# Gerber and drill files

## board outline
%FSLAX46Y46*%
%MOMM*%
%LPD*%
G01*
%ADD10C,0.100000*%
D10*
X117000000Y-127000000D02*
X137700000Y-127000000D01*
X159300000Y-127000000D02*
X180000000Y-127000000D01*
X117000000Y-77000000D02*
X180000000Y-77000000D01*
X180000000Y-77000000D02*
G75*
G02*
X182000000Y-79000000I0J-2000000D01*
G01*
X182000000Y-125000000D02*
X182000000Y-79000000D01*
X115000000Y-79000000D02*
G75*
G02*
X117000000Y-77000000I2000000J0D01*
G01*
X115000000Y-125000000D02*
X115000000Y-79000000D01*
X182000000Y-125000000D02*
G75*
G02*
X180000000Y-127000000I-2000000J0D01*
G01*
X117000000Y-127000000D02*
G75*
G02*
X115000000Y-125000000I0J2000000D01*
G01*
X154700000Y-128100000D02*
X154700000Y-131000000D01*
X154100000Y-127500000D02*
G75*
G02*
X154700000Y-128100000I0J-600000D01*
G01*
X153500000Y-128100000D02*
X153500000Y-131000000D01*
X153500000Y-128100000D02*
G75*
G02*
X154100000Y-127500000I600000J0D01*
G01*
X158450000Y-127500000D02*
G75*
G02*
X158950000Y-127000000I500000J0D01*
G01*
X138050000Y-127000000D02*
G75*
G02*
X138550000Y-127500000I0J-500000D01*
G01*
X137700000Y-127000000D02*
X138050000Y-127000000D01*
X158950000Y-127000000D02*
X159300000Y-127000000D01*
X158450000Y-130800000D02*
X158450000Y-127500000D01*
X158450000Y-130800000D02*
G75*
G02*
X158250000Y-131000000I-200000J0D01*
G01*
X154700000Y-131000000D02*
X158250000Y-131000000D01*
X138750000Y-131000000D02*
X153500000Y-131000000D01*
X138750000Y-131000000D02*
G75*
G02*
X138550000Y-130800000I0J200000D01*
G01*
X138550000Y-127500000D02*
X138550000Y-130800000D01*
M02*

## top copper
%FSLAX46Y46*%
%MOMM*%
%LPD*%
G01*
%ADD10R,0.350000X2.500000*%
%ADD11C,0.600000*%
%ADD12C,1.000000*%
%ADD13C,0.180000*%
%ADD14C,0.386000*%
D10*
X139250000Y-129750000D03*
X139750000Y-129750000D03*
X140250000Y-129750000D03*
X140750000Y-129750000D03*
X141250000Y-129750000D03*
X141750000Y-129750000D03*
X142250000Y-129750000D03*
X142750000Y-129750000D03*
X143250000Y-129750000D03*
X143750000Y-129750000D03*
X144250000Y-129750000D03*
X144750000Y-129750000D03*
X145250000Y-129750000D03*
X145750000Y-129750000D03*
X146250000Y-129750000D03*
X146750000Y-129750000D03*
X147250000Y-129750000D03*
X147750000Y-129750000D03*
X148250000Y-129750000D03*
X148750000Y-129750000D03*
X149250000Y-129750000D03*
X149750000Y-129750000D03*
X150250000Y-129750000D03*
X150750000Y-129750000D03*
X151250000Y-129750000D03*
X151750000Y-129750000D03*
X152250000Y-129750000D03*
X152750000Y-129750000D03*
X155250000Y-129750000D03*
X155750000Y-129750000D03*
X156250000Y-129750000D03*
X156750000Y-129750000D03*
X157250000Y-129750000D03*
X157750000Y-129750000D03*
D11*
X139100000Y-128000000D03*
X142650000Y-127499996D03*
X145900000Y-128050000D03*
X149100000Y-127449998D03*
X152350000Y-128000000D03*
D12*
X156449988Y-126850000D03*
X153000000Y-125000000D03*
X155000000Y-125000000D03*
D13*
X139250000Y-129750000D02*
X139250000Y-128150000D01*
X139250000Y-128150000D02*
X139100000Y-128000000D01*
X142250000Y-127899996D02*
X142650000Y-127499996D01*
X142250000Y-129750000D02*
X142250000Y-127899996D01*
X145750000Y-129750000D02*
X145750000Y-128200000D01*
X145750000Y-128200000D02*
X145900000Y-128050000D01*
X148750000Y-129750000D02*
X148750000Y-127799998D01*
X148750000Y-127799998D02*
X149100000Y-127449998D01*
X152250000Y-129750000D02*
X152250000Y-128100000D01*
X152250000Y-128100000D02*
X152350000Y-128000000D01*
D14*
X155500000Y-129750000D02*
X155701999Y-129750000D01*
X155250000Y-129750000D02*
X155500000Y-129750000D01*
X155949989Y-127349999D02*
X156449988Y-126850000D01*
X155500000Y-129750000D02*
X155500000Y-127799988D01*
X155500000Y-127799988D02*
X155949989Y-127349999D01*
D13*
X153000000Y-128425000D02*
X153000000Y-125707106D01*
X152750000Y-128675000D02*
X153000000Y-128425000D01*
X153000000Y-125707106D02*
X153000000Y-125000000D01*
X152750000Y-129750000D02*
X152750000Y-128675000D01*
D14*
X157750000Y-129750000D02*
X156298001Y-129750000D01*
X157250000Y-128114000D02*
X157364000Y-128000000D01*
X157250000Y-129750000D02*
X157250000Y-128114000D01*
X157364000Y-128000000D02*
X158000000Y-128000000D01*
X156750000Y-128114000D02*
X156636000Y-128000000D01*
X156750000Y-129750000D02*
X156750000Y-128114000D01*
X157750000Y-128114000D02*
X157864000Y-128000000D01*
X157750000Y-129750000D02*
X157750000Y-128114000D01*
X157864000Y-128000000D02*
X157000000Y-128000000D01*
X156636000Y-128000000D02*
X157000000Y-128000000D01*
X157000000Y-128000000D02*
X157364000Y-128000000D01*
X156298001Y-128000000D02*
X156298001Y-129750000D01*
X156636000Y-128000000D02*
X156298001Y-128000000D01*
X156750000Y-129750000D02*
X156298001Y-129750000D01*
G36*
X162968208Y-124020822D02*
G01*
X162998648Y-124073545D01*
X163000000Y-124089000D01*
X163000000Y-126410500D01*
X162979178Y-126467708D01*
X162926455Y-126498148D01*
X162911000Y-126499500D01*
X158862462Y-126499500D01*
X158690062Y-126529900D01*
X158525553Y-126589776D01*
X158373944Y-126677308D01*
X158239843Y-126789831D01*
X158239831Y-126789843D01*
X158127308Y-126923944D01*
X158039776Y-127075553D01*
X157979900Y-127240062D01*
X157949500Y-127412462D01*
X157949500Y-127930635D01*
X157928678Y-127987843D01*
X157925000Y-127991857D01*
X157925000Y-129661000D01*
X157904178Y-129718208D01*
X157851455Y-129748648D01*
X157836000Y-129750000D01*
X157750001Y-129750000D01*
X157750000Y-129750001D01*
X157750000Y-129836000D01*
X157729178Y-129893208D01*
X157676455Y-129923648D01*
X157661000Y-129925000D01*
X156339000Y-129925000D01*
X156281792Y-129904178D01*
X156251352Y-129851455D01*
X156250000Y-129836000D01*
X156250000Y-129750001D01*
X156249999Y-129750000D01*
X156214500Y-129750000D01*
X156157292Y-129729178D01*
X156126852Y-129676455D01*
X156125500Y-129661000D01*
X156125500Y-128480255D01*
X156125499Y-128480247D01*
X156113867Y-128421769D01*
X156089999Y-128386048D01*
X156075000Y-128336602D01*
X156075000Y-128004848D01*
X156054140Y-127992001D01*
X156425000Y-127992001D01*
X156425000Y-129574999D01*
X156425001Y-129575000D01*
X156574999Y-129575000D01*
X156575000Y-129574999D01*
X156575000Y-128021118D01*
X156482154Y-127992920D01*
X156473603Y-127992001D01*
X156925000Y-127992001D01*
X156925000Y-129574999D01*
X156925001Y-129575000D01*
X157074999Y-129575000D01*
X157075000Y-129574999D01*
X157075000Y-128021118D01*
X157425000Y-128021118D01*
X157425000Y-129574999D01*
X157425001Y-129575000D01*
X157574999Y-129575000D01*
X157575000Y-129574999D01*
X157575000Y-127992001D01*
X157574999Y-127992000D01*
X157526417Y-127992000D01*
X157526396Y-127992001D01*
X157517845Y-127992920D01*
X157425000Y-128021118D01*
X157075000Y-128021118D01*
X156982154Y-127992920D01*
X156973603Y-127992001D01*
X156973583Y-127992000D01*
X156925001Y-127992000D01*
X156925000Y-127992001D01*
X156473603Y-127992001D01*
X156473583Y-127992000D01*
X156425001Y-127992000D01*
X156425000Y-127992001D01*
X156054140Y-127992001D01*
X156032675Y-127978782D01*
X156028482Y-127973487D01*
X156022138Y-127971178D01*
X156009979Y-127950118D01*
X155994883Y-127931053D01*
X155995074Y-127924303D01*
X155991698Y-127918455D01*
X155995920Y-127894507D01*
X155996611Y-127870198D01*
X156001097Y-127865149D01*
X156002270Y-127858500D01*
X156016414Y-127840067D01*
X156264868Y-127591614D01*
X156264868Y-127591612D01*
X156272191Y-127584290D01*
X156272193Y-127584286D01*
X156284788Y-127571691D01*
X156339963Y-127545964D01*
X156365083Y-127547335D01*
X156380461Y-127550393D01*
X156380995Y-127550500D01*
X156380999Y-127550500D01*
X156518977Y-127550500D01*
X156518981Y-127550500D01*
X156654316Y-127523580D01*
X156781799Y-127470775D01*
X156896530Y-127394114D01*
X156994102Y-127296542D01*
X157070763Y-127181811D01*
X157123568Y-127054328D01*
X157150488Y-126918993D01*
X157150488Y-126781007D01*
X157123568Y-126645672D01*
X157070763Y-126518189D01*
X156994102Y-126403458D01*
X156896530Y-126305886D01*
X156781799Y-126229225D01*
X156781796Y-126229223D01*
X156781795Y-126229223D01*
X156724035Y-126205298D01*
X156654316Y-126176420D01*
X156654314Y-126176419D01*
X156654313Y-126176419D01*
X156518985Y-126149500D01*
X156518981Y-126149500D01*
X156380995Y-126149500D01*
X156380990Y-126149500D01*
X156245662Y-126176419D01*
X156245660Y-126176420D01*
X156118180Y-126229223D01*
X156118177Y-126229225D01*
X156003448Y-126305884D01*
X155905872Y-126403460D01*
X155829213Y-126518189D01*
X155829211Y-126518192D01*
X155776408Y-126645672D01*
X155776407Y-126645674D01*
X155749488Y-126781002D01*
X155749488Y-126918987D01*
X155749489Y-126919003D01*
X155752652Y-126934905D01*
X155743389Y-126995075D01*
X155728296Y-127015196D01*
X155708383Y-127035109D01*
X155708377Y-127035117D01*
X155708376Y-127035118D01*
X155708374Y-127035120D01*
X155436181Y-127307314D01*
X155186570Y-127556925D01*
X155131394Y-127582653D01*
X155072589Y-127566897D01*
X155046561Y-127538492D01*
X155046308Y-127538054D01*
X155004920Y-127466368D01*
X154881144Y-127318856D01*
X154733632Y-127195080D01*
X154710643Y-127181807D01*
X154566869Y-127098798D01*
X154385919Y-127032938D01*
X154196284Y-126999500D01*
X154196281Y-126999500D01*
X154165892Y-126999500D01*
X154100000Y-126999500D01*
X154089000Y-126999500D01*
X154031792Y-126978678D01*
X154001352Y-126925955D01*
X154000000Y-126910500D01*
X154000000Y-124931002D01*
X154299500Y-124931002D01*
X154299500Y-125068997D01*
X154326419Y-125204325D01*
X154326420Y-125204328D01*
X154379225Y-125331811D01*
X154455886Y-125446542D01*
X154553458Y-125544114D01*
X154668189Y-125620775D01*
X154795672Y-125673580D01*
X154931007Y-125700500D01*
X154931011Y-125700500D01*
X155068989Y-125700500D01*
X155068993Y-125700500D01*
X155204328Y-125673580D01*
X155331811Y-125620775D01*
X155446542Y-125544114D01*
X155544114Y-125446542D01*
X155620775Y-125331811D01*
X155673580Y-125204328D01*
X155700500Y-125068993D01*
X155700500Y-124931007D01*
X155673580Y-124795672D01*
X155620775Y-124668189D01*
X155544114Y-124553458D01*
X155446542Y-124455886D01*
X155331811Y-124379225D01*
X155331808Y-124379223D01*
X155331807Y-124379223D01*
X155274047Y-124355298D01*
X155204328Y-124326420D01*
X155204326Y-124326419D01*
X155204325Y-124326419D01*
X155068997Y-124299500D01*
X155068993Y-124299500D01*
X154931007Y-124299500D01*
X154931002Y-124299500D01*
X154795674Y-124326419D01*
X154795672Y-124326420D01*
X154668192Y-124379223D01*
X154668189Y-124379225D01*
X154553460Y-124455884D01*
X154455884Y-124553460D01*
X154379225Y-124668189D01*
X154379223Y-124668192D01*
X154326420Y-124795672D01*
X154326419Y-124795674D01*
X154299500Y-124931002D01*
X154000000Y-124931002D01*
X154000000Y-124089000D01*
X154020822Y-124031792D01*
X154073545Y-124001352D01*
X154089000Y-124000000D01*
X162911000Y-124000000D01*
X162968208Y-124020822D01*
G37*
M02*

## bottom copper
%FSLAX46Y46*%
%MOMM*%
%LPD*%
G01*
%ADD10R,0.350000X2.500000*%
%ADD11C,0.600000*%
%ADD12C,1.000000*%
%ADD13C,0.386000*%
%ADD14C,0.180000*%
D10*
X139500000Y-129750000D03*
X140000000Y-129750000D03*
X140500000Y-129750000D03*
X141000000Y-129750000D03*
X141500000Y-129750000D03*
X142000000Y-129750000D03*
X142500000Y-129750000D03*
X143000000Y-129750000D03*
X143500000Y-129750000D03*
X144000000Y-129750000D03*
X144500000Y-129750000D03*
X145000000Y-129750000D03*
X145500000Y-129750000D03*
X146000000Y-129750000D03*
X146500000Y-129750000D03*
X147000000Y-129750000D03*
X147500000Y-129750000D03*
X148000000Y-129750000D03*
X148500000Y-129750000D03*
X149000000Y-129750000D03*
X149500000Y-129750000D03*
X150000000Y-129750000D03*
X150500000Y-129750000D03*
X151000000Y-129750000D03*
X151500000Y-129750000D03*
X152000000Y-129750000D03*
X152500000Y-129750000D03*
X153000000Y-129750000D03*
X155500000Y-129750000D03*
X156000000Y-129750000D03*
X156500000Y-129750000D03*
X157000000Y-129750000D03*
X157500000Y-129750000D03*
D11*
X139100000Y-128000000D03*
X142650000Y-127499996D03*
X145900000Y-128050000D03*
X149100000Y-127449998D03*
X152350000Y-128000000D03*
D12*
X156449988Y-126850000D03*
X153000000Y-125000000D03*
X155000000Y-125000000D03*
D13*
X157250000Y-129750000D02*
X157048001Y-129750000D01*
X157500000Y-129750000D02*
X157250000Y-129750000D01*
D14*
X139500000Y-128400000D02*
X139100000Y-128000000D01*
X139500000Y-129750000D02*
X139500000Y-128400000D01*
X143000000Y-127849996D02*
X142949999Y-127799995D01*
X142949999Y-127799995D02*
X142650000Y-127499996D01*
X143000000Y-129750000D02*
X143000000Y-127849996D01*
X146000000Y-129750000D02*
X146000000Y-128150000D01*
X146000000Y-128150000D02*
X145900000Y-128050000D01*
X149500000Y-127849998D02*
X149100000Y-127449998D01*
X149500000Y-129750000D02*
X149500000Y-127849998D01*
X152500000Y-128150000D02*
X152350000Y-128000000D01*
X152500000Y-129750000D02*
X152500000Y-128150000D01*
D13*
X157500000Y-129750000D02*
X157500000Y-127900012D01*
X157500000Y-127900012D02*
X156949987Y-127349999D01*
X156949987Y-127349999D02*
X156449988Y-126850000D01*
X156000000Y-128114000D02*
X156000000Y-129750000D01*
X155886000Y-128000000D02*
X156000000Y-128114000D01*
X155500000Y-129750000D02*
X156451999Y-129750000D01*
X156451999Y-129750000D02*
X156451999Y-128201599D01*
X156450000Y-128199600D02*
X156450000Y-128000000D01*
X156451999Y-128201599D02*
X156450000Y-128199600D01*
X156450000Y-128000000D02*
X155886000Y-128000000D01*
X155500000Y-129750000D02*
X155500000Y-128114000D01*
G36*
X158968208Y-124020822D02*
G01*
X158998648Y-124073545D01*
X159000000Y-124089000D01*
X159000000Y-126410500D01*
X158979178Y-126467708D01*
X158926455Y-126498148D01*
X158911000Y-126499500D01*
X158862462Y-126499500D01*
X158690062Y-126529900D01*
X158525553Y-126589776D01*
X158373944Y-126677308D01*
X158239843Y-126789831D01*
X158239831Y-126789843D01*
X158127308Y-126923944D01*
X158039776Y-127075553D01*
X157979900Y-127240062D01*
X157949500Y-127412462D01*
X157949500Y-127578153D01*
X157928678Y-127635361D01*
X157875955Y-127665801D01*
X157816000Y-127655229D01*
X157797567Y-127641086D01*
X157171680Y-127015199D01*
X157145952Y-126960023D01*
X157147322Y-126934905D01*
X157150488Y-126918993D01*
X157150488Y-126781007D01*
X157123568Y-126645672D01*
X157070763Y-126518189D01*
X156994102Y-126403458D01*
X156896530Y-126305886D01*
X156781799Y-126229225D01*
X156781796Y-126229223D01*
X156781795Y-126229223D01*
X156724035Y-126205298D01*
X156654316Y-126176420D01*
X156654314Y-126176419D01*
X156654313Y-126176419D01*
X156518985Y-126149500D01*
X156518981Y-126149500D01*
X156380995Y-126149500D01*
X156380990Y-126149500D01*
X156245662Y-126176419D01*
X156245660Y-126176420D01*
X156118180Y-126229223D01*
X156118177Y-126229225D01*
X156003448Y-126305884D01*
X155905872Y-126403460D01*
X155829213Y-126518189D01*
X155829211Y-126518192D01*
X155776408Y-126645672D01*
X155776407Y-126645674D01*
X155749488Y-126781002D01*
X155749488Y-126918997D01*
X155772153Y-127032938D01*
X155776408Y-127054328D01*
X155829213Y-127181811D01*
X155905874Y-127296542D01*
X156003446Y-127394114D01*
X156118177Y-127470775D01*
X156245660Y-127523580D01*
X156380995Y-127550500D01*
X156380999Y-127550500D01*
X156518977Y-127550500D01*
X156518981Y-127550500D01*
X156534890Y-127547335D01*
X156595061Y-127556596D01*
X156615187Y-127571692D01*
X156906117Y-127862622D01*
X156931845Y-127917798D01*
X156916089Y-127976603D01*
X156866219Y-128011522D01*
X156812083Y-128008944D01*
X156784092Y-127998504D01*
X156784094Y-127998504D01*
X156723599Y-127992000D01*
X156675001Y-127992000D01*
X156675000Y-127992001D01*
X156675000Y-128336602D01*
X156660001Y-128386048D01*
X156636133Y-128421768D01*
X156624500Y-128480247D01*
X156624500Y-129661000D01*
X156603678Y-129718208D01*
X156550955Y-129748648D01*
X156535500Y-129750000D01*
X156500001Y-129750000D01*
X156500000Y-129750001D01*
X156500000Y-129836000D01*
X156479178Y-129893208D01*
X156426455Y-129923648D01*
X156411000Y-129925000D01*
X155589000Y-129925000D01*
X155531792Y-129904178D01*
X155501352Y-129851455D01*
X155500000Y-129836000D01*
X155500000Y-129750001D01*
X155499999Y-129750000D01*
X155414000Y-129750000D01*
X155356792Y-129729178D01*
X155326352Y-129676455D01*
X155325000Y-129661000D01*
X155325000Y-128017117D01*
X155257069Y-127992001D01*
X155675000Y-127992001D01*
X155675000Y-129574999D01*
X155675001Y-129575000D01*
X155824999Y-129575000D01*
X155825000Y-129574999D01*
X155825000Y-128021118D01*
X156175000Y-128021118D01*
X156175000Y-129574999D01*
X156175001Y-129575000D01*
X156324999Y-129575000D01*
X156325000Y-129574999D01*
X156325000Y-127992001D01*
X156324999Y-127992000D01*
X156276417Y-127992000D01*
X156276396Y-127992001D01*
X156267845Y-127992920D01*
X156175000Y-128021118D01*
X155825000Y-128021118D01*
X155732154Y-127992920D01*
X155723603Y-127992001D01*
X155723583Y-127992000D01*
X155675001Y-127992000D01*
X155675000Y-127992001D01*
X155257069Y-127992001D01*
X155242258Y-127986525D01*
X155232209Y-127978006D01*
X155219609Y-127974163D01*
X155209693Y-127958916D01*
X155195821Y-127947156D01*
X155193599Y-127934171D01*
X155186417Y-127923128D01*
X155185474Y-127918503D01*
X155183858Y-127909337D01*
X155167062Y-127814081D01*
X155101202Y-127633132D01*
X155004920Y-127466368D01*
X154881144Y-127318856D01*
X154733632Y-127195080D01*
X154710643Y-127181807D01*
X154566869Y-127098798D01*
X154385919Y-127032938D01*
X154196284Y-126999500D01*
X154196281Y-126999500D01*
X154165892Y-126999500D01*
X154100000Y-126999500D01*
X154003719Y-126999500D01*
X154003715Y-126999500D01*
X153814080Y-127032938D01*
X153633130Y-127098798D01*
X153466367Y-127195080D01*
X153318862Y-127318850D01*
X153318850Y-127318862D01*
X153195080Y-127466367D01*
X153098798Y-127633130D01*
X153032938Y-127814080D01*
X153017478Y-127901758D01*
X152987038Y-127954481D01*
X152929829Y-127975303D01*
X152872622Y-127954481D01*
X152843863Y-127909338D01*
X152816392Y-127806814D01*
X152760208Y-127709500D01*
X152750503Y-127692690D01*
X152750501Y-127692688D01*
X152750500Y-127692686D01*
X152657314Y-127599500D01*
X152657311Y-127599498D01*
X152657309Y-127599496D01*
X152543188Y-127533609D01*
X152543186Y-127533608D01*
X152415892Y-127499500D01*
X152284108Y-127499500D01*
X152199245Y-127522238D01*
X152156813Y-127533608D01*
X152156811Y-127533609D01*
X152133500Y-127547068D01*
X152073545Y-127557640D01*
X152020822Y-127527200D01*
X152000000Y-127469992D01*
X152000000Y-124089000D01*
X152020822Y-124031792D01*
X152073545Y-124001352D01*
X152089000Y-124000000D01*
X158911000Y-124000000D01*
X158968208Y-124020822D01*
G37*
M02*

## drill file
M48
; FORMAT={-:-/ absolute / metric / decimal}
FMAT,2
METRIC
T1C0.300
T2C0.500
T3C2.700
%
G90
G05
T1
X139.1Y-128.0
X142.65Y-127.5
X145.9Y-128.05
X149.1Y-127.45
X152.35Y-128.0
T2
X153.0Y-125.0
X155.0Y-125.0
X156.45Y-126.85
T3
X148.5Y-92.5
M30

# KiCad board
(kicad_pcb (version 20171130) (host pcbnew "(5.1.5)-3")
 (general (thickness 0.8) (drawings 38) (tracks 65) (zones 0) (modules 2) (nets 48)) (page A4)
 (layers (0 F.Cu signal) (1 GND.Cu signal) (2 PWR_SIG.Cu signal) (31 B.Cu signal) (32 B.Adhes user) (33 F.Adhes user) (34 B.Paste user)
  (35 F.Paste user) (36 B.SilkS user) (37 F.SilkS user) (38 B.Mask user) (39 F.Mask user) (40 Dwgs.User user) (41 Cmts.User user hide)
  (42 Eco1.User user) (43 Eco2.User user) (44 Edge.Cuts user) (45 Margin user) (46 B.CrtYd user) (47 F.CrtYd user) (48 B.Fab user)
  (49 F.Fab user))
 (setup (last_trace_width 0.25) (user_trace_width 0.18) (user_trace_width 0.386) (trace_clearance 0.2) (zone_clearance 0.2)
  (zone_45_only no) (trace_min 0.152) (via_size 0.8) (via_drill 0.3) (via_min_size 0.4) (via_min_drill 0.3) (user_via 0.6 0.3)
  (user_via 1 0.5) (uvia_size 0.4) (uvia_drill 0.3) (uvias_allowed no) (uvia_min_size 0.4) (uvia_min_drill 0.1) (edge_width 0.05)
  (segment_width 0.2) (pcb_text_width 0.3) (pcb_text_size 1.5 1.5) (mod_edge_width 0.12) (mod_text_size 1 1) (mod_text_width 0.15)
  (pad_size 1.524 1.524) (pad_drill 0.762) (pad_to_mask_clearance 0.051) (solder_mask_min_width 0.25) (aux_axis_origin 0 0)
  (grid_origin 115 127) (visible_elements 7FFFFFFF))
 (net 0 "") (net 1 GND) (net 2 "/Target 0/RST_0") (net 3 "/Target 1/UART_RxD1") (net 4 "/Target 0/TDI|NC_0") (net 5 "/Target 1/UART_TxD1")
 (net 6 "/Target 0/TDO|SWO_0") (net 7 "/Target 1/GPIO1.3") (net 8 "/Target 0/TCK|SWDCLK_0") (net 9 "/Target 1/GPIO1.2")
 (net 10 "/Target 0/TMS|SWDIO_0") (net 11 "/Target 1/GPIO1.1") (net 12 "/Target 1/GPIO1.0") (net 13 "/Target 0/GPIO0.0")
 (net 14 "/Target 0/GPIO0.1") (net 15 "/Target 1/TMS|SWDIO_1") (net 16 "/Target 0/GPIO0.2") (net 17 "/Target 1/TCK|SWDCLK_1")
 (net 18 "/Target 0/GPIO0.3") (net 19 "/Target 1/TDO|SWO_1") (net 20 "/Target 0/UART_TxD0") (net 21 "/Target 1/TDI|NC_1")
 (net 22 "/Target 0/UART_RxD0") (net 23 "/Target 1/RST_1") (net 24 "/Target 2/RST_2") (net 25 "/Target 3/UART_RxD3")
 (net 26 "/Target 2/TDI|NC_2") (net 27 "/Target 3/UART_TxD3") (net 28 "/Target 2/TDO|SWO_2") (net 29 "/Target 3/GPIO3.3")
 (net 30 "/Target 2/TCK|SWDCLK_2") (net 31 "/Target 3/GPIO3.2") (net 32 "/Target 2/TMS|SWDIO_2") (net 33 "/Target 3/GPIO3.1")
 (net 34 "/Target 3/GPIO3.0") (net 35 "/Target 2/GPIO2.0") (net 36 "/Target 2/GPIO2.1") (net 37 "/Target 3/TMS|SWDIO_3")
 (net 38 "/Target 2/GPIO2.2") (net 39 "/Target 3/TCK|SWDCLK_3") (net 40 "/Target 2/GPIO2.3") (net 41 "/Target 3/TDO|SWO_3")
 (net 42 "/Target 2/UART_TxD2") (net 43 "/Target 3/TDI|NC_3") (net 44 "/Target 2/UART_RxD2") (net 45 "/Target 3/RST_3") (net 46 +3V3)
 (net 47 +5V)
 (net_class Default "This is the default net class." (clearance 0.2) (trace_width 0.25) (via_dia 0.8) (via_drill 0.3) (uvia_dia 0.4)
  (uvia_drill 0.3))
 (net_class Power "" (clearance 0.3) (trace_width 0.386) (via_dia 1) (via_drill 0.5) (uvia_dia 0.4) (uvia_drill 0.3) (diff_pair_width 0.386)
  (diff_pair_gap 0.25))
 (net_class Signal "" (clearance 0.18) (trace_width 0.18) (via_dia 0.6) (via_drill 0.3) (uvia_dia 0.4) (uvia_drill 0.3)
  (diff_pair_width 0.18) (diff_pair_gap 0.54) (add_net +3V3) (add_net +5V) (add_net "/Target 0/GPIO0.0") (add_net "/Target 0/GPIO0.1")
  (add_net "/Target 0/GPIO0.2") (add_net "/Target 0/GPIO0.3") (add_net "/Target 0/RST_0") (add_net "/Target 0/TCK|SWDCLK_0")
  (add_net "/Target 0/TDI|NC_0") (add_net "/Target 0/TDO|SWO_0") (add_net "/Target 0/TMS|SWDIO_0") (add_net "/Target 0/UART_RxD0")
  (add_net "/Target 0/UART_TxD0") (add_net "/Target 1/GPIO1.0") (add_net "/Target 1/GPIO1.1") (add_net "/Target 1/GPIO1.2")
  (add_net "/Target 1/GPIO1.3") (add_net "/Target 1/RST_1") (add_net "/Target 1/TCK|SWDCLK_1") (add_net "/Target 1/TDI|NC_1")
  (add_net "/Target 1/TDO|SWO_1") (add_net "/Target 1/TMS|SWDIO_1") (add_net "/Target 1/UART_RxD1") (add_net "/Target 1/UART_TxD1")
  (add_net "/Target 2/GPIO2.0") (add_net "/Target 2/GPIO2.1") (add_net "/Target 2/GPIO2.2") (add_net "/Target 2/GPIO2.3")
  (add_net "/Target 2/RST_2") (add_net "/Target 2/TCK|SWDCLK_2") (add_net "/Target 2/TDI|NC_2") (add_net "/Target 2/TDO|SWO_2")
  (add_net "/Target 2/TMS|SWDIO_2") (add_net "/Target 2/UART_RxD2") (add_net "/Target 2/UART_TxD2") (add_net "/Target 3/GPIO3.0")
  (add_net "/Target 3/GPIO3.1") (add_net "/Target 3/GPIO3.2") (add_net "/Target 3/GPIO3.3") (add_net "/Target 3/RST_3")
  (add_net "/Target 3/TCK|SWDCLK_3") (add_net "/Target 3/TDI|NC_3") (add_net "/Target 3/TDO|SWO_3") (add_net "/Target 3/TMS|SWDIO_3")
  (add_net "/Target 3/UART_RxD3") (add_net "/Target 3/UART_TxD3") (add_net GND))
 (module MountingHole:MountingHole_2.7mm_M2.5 (layer F.Cu) (at 148.5 92.5)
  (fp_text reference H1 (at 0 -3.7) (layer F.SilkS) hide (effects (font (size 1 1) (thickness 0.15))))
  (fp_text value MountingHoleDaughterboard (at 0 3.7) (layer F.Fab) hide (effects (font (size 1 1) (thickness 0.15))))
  (pad 1 np_thru_hole circle (at 0 0) (size 2.7 2.7) (drill 2.7) (layers *.Cu *.Mask)))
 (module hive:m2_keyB (layer F.Cu) (at 148.5 131)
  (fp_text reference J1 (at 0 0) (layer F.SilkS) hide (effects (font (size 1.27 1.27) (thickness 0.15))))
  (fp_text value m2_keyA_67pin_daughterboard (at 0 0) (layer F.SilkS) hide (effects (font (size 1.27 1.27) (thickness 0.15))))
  (fp_line (start 6.2 -2.9) (end 6.2 0) (layer Edge.Cuts) (width 0.1))
  (fp_arc (start 5.6 -2.9) (end 5.6 -3.5) (angle 90) (layer Edge.Cuts) (width 0.1))
  (fp_line (start 5 -2.9) (end 5 0) (layer Edge.Cuts) (width 0.1))
  (fp_arc (start 5.6 -2.9) (end 5.6 -3.5) (angle -90) (layer Edge.Cuts) (width 0.1))
  (fp_arc (start 10.45 -3.5) (end 9.95 -3.5) (angle 90) (layer Edge.Cuts) (width 0.1))
  (fp_arc (start -10.45 -3.5) (end -10.45 -4) (angle 90) (layer Edge.Cuts) (width 0.1))
  (fp_line (start -10.8 -4) (end -10.45 -4) (layer Edge.Cuts) (width 0.1))
  (fp_line (start 10.45 -4) (end 10.8 -4) (layer Edge.Cuts) (width 0.1))
  (fp_line (start 9.95 -0.2) (end 9.95 -3.5) (layer Edge.Cuts) (width 0.1))
  (fp_arc (start 9.75 -0.2) (end 9.75 0) (angle -90) (layer Edge.Cuts) (width 0.1))
  (fp_line (start 6.2 0) (end 9.75 0) (layer Edge.Cuts) (width 0.1))
  (fp_line (start -9.75 0) (end 5 0) (layer Edge.Cuts) (width 0.1))
  (fp_arc (start -9.75 -0.2) (end -9.95 -0.2) (angle -90) (layer Edge.Cuts) (width 0.1))
  (fp_line (start -9.95 -3.5) (end -9.95 -0.2) (layer Edge.Cuts) (width 0.1))
  (pad 75 smd rect (at -9.25 -1.25) (size 0.35 2.5) (layers F.Cu F.Paste F.Mask) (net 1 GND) (solder_mask_margin 0.1016))
  (pad 74 smd rect (at -9 -1.25) (size 0.35 2.5) (layers B.Cu B.Paste B.Mask) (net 1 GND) (solder_mask_margin 0.1016))
  (pad 73 smd rect (at -8.75 -1.25) (size 0.35 2.5) (layers F.Cu F.Paste F.Mask) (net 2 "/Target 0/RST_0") (solder_mask_margin 0.1016))
  (pad 72 smd rect (at -8.5 -1.25) (size 0.35 2.5) (layers B.Cu B.Paste B.Mask) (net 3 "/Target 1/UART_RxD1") (solder_mask_margin 0.1016))
  (pad 71 smd rect (at -8.25 -1.25) (size 0.35 2.5) (layers F.Cu F.Paste F.Mask) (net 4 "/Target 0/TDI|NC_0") (solder_mask_margin 0.1016))
  (pad 70 smd rect (at -8 -1.25) (size 0.35 2.5) (layers B.Cu B.Paste B.Mask) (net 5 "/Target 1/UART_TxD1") (solder_mask_margin 0.1016))
  (pad 69 smd rect (at -7.75 -1.25) (size 0.35 2.5) (layers F.Cu F.Paste F.Mask) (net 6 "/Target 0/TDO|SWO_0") (solder_mask_margin 0.1016))
  (pad 68 smd rect (at -7.5 -1.25) (size 0.35 2.5) (layers B.Cu B.Paste B.Mask) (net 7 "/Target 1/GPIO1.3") (solder_mask_margin 0.1016))
  (pad 67 smd rect (at -7.25 -1.25) (size 0.35 2.5) (layers F.Cu F.Paste F.Mask) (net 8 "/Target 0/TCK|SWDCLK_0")
   (solder_mask_margin 0.1016))
  (pad 66 smd rect (at -7 -1.25) (size 0.35 2.5) (layers B.Cu B.Paste B.Mask) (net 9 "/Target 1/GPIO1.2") (solder_mask_margin 0.1016))
  (pad 65 smd rect (at -6.75 -1.25) (size 0.35 2.5) (layers F.Cu F.Paste F.Mask) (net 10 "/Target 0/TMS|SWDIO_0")
   (solder_mask_margin 0.1016))
  (pad 64 smd rect (at -6.5 -1.25) (size 0.35 2.5) (layers B.Cu B.Paste B.Mask) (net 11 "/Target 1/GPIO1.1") (solder_mask_margin 0.1016))
  (pad 63 smd rect (at -6.25 -1.25) (size 0.35 2.5) (layers F.Cu F.Paste F.Mask) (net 1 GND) (solder_mask_margin 0.1016))
  (pad 62 smd rect (at -6 -1.25) (size 0.35 2.5) (layers B.Cu B.Paste B.Mask) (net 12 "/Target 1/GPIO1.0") (solder_mask_margin 0.1016))
  (pad 61 smd rect (at -5.75 -1.25) (size 0.35 2.5) (layers F.Cu F.Paste F.Mask) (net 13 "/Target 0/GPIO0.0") (solder_mask_margin 0.1016))
  (pad 60 smd rect (at -5.5 -1.25) (size 0.35 2.5) (layers B.Cu B.Paste B.Mask) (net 1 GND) (solder_mask_margin 0.1016))
  (pad 59 smd rect (at -5.25 -1.25) (size 0.35 2.5) (layers F.Cu F.Paste F.Mask) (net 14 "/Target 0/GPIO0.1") (solder_mask_margin 0.1016))
  (pad 58 smd rect (at -5 -1.25) (size 0.35 2.5) (layers B.Cu B.Paste B.Mask) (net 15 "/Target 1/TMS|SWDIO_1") (solder_mask_margin 0.1016))
  (pad 57 smd rect (at -4.75 -1.25) (size 0.35 2.5) (layers F.Cu F.Paste F.Mask) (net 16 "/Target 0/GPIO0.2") (solder_mask_margin 0.1016))
  (pad 56 smd rect (at -4.5 -1.25) (size 0.35 2.5) (layers B.Cu B.Paste B.Mask) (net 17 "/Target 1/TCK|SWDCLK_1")
   (solder_mask_margin 0.1016))
  (pad 55 smd rect (at -4.25 -1.25) (size 0.35 2.5) (layers F.Cu F.Paste F.Mask) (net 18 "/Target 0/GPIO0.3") (solder_mask_margin 0.1016))
  (pad 54 smd rect (at -4 -1.25) (size 0.35 2.5) (layers B.Cu B.Paste B.Mask) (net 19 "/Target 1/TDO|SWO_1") (solder_mask_margin 0.1016))
  (pad 53 smd rect (at -3.75 -1.25) (size 0.35 2.5) (layers F.Cu F.Paste F.Mask) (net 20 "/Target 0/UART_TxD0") (solder_mask_margin 0.1016))
  (pad 52 smd rect (at -3.5 -1.25) (size 0.35 2.5) (layers B.Cu B.Paste B.Mask) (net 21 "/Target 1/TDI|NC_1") (solder_mask_margin 0.1016))
  (pad 51 smd rect (at -3.25 -1.25) (size 0.35 2.5) (layers F.Cu F.Paste F.Mask) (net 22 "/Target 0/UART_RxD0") (solder_mask_margin 0.1016))
  (pad 50 smd rect (at -3 -1.25) (size 0.35 2.5) (layers B.Cu B.Paste B.Mask) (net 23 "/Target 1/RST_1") (solder_mask_margin 0.1016))
  (pad 49 smd rect (at -2.75 -1.25) (size 0.35 2.5) (layers F.Cu F.Paste F.Mask) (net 1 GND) (solder_mask_margin 0.1016))
  (pad 48 smd rect (at -2.5 -1.25) (size 0.35 2.5) (layers B.Cu B.Paste B.Mask) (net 1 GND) (solder_mask_margin 0.1016))
  (pad 47 smd rect (at -2.25 -1.25) (size 0.35 2.5) (layers F.Cu F.Paste F.Mask) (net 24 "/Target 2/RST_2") (solder_mask_margin 0.1016))
  (pad 46 smd rect (at -2 -1.25) (size 0.35 2.5) (layers B.Cu B.Paste B.Mask) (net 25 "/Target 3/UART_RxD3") (solder_mask_margin 0.1016))
  (pad 45 smd rect (at -1.75 -1.25) (size 0.35 2.5) (layers F.Cu F.Paste F.Mask) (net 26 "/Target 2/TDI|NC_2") (solder_mask_margin 0.1016))
  (pad 44 smd rect (at -1.5 -1.25) (size 0.35 2.5) (layers B.Cu B.Paste B.Mask) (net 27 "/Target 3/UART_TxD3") (solder_mask_margin 0.1016))
  (pad 43 smd rect (at -1.25 -1.25) (size 0.35 2.5) (layers F.Cu F.Paste F.Mask) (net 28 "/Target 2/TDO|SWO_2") (solder_mask_margin 0.1016))
  (pad 42 smd rect (at -1 -1.25) (size 0.35 2.5) (layers B.Cu B.Paste B.Mask) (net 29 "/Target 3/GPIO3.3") (solder_mask_margin 0.1016))
  (pad 41 smd rect (at -0.75 -1.25) (size 0.35 2.5) (layers F.Cu F.Paste F.Mask) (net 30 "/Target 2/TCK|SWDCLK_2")
   (solder_mask_margin 0.1016))
  (pad 40 smd rect (at -0.5 -1.25) (size 0.35 2.5) (layers B.Cu B.Paste B.Mask) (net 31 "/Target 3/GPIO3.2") (solder_mask_margin 0.1016))
  (pad 39 smd rect (at -0.25 -1.25) (size 0.35 2.5) (layers F.Cu F.Paste F.Mask) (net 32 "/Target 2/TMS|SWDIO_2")
   (solder_mask_margin 0.1016))
  (pad 38 smd rect (at 0 -1.25) (size 0.35 2.5) (layers B.Cu B.Paste B.Mask) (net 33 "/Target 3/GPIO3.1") (solder_mask_margin 0.1016))
  (pad 37 smd rect (at 0.25 -1.25) (size 0.35 2.5) (layers F.Cu F.Paste F.Mask) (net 1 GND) (solder_mask_margin 0.1016))
  (pad 36 smd rect (at 0.5 -1.25) (size 0.35 2.5) (layers B.Cu B.Paste B.Mask) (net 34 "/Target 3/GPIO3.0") (solder_mask_margin 0.1016))
  (pad 35 smd rect (at 0.75 -1.25) (size 0.35 2.5) (layers F.Cu F.Paste F.Mask) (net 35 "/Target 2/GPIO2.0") (solder_mask_margin 0.1016))
  (pad 34 smd rect (at 1 -1.25) (size 0.35 2.5) (layers B.Cu B.Paste B.Mask) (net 1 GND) (solder_mask_margin 0.1016))
  (pad 33 smd rect (at 1.25 -1.25) (size 0.35 2.5) (layers F.Cu F.Paste F.Mask) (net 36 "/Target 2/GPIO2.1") (solder_mask_margin 0.1016))
  (pad 32 smd rect (at 1.5 -1.25) (size 0.35 2.5) (layers B.Cu B.Paste B.Mask) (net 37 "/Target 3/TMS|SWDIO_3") (solder_mask_margin 0.1016))
  (pad 31 smd rect (at 1.75 -1.25) (size 0.35 2.5) (layers F.Cu F.Paste F.Mask) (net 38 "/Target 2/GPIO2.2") (solder_mask_margin 0.1016))
  (pad 30 smd rect (at 2 -1.25) (size 0.35 2.5) (layers B.Cu B.Paste B.Mask) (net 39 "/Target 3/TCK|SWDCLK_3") (solder_mask_margin 0.1016))
  (pad 29 smd rect (at 2.25 -1.25) (size 0.35 2.5) (layers F.Cu F.Paste F.Mask) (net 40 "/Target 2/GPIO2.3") (solder_mask_margin 0.1016))
  (pad 28 smd rect (at 2.5 -1.25) (size 0.35 2.5) (layers B.Cu B.Paste B.Mask) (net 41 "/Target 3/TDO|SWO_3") (solder_mask_margin 0.1016))
  (pad 27 smd rect (at 2.75 -1.25) (size 0.35 2.5) (layers F.Cu F.Paste F.Mask) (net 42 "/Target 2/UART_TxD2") (solder_mask_margin 0.1016))
  (pad 26 smd rect (at 3 -1.25) (size 0.35 2.5) (layers B.Cu B.Paste B.Mask) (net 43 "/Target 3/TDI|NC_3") (solder_mask_margin 0.1016))
  (pad 25 smd rect (at 3.25 -1.25) (size 0.35 2.5) (layers F.Cu F.Paste F.Mask) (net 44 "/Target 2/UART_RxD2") (solder_mask_margin 0.1016))
  (pad 24 smd rect (at 3.5 -1.25) (size 0.35 2.5) (layers B.Cu B.Paste B.Mask) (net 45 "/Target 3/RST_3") (solder_mask_margin 0.1016))
  (pad 23 smd rect (at 3.75 -1.25) (size 0.35 2.5) (layers F.Cu F.Paste F.Mask) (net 1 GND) (solder_mask_margin 0.1016))
  (pad 22 smd rect (at 4 -1.25) (size 0.35 2.5) (layers B.Cu B.Paste B.Mask) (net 1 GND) (solder_mask_margin 0.1016))
  (pad 21 smd rect (at 4.25 -1.25) (size 0.35 2.5) (layers F.Cu F.Paste F.Mask) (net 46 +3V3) (solder_mask_margin 0.1016))
  (pad 20 smd rect (at 4.5 -1.25) (size 0.35 2.5) (layers B.Cu B.Paste B.Mask) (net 46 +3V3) (solder_mask_margin 0.1016))
  (pad 11 smd rect (at 6.75 -1.25) (size 0.35 2.5) (layers F.Cu F.Paste F.Mask) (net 1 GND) (solder_mask_margin 0.1016))
  (pad 10 smd rect (at 7 -1.25) (size 0.35 2.5) (layers B.Cu B.Paste B.Mask) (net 46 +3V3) (solder_mask_margin 0.1016))
  (pad 9 smd rect (at 7.25 -1.25) (size 0.35 2.5) (layers F.Cu F.Paste F.Mask) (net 1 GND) (solder_mask_margin 0.1016))
  (pad 8 smd rect (at 7.5 -1.25) (size 0.35 2.5) (layers B.Cu B.Paste B.Mask) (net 46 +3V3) (solder_mask_margin 0.1016))
  (pad 7 smd rect (at 7.75 -1.25) (size 0.35 2.5) (layers F.Cu F.Paste F.Mask) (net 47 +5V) (solder_mask_margin 0.1016))
  (pad 6 smd rect (at 8 -1.25) (size 0.35 2.5) (layers B.Cu B.Paste B.Mask) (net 46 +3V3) (solder_mask_margin 0.1016))
  (pad 5 smd rect (at 8.25 -1.25) (size 0.35 2.5) (layers F.Cu F.Paste F.Mask) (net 47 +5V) (solder_mask_margin 0.1016))
  (pad 4 smd rect (at 8.5 -1.25) (size 0.35 2.5) (layers B.Cu B.Paste B.Mask) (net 1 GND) (solder_mask_margin 0.1016))
  (pad 3 smd rect (at 8.75 -1.25) (size 0.35 2.5) (layers F.Cu F.Paste F.Mask) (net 47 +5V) (solder_mask_margin 0.1016))
  (pad 2 smd rect (at 9 -1.25) (size 0.35 2.5) (layers B.Cu B.Paste B.Mask) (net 1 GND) (solder_mask_margin 0.1016))
  (pad 1 smd rect (at 9.25 -1.25) (size 0.35 2.5) (layers F.Cu F.Paste F.Mask) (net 47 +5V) (solder_mask_margin 0.1016)))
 (gr_line (start 117 127) (end 137.7 127) (layer Edge.Cuts) (width 0.1))
 (gr_line (start 159.3 127) (end 180 127) (layer Edge.Cuts) (width 0.1))
 (gr_line (start 117 77) (end 180 77) (layer Edge.Cuts) (width 0.1))
 (gr_arc (start 180 79) (end 182 79) (angle -90) (layer Edge.Cuts) (width 0.1))
 (gr_line (start 182 125) (end 182 79) (layer Edge.Cuts) (width 0.1))
 (gr_arc (start 117 79) (end 117 77) (angle -90) (layer Edge.Cuts) (width 0.1))
 (gr_line (start 115 125) (end 115 79) (layer Edge.Cuts) (width 0.1))
 (gr_arc (start 180 125) (end 180 127) (angle -90) (layer Edge.Cuts) (width 0.1))
 (gr_arc (start 117 125) (end 115 125) (angle -90) (layer Edge.Cuts) (width 0.1))
 (segment (start 157.25 129.75) (end 157.048001 129.75) (width 0.386) (layer B.Cu) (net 1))
 (segment (start 157.5 129.75) (end 157.25 129.75) (width 0.386) (layer B.Cu) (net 1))
 (via (at 139.1 128) (size 0.6) (drill 0.3) (layers F.Cu B.Cu) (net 1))
 (segment (start 139.25 129.75) (end 139.25 128.15) (width 0.18) (layer F.Cu) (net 1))
 (segment (start 139.25 128.15) (end 139.1 128) (width 0.18) (layer F.Cu) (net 1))
 (segment (start 139.5 128.4) (end 139.1 128) (width 0.18) (layer B.Cu) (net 1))
 (segment (start 139.5 129.75) (end 139.5 128.4) (width 0.18) (layer B.Cu) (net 1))
 (segment (start 143 127.849996) (end 142.949999 127.799995) (width 0.18) (layer B.Cu) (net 1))
 (segment (start 142.949999 127.799995) (end 142.65 127.499996) (width 0.18) (layer B.Cu) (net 1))
 (via (at 142.65 127.499996) (size 0.6) (drill 0.3) (layers F.Cu B.Cu) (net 1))
 (segment (start 143 129.75) (end 143 127.849996) (width 0.18) (layer B.Cu) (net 1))
 (segment (start 142.25 127.899996) (end 142.65 127.499996) (width 0.18) (layer F.Cu) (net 1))
 (segment (start 142.25 129.75) (end 142.25 127.899996) (width 0.18) (layer F.Cu) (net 1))
 (via (at 145.9 128.05) (size 0.6) (drill 0.3) (layers F.Cu B.Cu) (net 1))
 (segment (start 146 129.75) (end 146 128.15) (width 0.18) (layer B.Cu) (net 1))
 (segment (start 145.75 129.75) (end 145.75 128.2) (width 0.18) (layer F.Cu) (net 1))
 (segment (start 146 128.15) (end 145.9 128.05) (width 0.18) (layer B.Cu) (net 1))
 (segment (start 145.75 128.2) (end 145.9 128.05) (width 0.18) (layer F.Cu) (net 1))
 (via (at 149.1 127.449998) (size 0.6) (drill 0.3) (layers F.Cu B.Cu) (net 1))
 (segment (start 149.5 127.849998) (end 149.1 127.449998) (width 0.18) (layer B.Cu) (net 1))
 (segment (start 148.75 129.75) (end 148.75 127.799998) (width 0.18) (layer F.Cu) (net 1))
 (segment (start 149.5 129.75) (end 149.5 127.849998) (width 0.18) (layer B.Cu) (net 1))
 (segment (start 148.75 127.799998) (end 149.1 127.449998) (width 0.18) (layer F.Cu) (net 1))
 (segment (start 152.25 129.75) (end 152.25 128.1) (width 0.18) (layer F.Cu) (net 1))
 (segment (start 152.5 128.15) (end 152.35 128) (width 0.18) (layer B.Cu) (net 1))
 (segment (start 152.5 129.75) (end 152.5 128.15) (width 0.18) (layer B.Cu) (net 1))
 (via (at 152.35 128) (size 0.6) (drill 0.3) (layers F.Cu B.Cu) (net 1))
 (segment (start 152.25 128.1) (end 152.35 128) (width 0.18) (layer F.Cu) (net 1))
 (segment (start 155.5 129.75) (end 155.701999 129.75) (width 0.386) (layer F.Cu) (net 1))
 (segment (start 155.25 129.75) (end 155.5 129.75) (width 0.386) (layer F.Cu) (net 1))
 (via (at 156.449988 126.85) (size 1) (drill 0.5) (layers F.Cu B.Cu) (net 1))
 (segment (start 157.5 129.75) (end 157.5 127.900012) (width 0.386) (layer B.Cu) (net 1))
 (segment (start 157.5 127.900012) (end 156.949987 127.349999) (width 0.386) (layer B.Cu) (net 1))
 (segment (start 156.949987 127.349999) (end 156.449988 126.85) (width 0.386) (layer B.Cu) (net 1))
 (segment (start 155.949989 127.349999) (end 156.449988 126.85) (width 0.386) (layer F.Cu) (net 1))
 (segment (start 155.5 129.75) (end 155.5 127.799988) (width 0.386) (layer F.Cu) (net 1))
 (segment (start 155.5 127.799988) (end 155.949989 127.349999) (width 0.386) (layer F.Cu) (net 1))
 (via (at 153 125) (size 1) (drill 0.5) (layers F.Cu B.Cu) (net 46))
 (segment (start 156 128.114) (end 156 129.75) (width 0.386) (layer B.Cu) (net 46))
 (segment (start 155.886 128) (end 156 128.114) (width 0.386) (layer B.Cu) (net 46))
 (segment (start 155.5 129.75) (end 156.451999 129.75) (width 0.386) (layer B.Cu) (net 46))
 (segment (start 156.451999 129.75) (end 156.451999 128.201599) (width 0.386) (layer B.Cu) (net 46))
 (segment (start 156.45 128.1996) (end 156.45 128) (width 0.386) (layer B.Cu) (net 46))
 (segment (start 156.451999 128.201599) (end 156.45 128.1996) (width 0.386) (layer B.Cu) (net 46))
 (segment (start 156.45 128) (end 155.886 128) (width 0.386) (layer B.Cu) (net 46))
 (segment (start 155.5 129.75) (end 155.5 128.114) (width 0.386) (layer B.Cu) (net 46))
 (via (at 155 125) (size 1) (drill 0.5) (layers F.Cu B.Cu) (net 46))
 (segment (start 153 128.425) (end 153 125.707106) (width 0.18) (layer F.Cu) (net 46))
 (segment (start 152.75 128.675) (end 153 128.425) (width 0.18) (layer F.Cu) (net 46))
 (segment (start 153 125.707106) (end 153 125) (width 0.18) (layer F.Cu) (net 46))
 (segment (start 152.75 129.75) (end 152.75 128.675) (width 0.18) (layer F.Cu) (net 46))
 (segment (start 157.75 129.75) (end 156.298001 129.75) (width 0.386) (layer F.Cu) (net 47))
 (segment (start 157.25 128.114) (end 157.364 128) (width 0.386) (layer F.Cu) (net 47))
 (segment (start 157.25 129.75) (end 157.25 128.114) (width 0.386) (layer F.Cu) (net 47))
 (segment (start 157.364 128) (end 158 128) (width 0.386) (layer F.Cu) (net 47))
 (segment (start 156.75 128.114) (end 156.636 128) (width 0.386) (layer F.Cu) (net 47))
 (segment (start 156.75 129.75) (end 156.75 128.114) (width 0.386) (layer F.Cu) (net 47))
 (segment (start 157.75 128.114) (end 157.864 128) (width 0.386) (layer F.Cu) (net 47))
 (segment (start 157.75 129.75) (end 157.75 128.114) (width 0.386) (layer F.Cu) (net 47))
 (segment (start 157.864 128) (end 157 128) (width 0.386) (layer F.Cu) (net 47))
 (segment (start 156.636 128) (end 157 128) (width 0.386) (layer F.Cu) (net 47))
 (segment (start 157 128) (end 157.364 128) (width 0.386) (layer F.Cu) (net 47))
 (segment (start 156.298001 128) (end 156.298001 129.75) (width 0.386) (layer F.Cu) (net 47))
 (segment (start 156.636 128) (end 156.298001 128) (width 0.386) (layer F.Cu) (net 47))
 (segment (start 156.75 129.75) (end 156.298001 129.75) (width 0.386) (layer F.Cu) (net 47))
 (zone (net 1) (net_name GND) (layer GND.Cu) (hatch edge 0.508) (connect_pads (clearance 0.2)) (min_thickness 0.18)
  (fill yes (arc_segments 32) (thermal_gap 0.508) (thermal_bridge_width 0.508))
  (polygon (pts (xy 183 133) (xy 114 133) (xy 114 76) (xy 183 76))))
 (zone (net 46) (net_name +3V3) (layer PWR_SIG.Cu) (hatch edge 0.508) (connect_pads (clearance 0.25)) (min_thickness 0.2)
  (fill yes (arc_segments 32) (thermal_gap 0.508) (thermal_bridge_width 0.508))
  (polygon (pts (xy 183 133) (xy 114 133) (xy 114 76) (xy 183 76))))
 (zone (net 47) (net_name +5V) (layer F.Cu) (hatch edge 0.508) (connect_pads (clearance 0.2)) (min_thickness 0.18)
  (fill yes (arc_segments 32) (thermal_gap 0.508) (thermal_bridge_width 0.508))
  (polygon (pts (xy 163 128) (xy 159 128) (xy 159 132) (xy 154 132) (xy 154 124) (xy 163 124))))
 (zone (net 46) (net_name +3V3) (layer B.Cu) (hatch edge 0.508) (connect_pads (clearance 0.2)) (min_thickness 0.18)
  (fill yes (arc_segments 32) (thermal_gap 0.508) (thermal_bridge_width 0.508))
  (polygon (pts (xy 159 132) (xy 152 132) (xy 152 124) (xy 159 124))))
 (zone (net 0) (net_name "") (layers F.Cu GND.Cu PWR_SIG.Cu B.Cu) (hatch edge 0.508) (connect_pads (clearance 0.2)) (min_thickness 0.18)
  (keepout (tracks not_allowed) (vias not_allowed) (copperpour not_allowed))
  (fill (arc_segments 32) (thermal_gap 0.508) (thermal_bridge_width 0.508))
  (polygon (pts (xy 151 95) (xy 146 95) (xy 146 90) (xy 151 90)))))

